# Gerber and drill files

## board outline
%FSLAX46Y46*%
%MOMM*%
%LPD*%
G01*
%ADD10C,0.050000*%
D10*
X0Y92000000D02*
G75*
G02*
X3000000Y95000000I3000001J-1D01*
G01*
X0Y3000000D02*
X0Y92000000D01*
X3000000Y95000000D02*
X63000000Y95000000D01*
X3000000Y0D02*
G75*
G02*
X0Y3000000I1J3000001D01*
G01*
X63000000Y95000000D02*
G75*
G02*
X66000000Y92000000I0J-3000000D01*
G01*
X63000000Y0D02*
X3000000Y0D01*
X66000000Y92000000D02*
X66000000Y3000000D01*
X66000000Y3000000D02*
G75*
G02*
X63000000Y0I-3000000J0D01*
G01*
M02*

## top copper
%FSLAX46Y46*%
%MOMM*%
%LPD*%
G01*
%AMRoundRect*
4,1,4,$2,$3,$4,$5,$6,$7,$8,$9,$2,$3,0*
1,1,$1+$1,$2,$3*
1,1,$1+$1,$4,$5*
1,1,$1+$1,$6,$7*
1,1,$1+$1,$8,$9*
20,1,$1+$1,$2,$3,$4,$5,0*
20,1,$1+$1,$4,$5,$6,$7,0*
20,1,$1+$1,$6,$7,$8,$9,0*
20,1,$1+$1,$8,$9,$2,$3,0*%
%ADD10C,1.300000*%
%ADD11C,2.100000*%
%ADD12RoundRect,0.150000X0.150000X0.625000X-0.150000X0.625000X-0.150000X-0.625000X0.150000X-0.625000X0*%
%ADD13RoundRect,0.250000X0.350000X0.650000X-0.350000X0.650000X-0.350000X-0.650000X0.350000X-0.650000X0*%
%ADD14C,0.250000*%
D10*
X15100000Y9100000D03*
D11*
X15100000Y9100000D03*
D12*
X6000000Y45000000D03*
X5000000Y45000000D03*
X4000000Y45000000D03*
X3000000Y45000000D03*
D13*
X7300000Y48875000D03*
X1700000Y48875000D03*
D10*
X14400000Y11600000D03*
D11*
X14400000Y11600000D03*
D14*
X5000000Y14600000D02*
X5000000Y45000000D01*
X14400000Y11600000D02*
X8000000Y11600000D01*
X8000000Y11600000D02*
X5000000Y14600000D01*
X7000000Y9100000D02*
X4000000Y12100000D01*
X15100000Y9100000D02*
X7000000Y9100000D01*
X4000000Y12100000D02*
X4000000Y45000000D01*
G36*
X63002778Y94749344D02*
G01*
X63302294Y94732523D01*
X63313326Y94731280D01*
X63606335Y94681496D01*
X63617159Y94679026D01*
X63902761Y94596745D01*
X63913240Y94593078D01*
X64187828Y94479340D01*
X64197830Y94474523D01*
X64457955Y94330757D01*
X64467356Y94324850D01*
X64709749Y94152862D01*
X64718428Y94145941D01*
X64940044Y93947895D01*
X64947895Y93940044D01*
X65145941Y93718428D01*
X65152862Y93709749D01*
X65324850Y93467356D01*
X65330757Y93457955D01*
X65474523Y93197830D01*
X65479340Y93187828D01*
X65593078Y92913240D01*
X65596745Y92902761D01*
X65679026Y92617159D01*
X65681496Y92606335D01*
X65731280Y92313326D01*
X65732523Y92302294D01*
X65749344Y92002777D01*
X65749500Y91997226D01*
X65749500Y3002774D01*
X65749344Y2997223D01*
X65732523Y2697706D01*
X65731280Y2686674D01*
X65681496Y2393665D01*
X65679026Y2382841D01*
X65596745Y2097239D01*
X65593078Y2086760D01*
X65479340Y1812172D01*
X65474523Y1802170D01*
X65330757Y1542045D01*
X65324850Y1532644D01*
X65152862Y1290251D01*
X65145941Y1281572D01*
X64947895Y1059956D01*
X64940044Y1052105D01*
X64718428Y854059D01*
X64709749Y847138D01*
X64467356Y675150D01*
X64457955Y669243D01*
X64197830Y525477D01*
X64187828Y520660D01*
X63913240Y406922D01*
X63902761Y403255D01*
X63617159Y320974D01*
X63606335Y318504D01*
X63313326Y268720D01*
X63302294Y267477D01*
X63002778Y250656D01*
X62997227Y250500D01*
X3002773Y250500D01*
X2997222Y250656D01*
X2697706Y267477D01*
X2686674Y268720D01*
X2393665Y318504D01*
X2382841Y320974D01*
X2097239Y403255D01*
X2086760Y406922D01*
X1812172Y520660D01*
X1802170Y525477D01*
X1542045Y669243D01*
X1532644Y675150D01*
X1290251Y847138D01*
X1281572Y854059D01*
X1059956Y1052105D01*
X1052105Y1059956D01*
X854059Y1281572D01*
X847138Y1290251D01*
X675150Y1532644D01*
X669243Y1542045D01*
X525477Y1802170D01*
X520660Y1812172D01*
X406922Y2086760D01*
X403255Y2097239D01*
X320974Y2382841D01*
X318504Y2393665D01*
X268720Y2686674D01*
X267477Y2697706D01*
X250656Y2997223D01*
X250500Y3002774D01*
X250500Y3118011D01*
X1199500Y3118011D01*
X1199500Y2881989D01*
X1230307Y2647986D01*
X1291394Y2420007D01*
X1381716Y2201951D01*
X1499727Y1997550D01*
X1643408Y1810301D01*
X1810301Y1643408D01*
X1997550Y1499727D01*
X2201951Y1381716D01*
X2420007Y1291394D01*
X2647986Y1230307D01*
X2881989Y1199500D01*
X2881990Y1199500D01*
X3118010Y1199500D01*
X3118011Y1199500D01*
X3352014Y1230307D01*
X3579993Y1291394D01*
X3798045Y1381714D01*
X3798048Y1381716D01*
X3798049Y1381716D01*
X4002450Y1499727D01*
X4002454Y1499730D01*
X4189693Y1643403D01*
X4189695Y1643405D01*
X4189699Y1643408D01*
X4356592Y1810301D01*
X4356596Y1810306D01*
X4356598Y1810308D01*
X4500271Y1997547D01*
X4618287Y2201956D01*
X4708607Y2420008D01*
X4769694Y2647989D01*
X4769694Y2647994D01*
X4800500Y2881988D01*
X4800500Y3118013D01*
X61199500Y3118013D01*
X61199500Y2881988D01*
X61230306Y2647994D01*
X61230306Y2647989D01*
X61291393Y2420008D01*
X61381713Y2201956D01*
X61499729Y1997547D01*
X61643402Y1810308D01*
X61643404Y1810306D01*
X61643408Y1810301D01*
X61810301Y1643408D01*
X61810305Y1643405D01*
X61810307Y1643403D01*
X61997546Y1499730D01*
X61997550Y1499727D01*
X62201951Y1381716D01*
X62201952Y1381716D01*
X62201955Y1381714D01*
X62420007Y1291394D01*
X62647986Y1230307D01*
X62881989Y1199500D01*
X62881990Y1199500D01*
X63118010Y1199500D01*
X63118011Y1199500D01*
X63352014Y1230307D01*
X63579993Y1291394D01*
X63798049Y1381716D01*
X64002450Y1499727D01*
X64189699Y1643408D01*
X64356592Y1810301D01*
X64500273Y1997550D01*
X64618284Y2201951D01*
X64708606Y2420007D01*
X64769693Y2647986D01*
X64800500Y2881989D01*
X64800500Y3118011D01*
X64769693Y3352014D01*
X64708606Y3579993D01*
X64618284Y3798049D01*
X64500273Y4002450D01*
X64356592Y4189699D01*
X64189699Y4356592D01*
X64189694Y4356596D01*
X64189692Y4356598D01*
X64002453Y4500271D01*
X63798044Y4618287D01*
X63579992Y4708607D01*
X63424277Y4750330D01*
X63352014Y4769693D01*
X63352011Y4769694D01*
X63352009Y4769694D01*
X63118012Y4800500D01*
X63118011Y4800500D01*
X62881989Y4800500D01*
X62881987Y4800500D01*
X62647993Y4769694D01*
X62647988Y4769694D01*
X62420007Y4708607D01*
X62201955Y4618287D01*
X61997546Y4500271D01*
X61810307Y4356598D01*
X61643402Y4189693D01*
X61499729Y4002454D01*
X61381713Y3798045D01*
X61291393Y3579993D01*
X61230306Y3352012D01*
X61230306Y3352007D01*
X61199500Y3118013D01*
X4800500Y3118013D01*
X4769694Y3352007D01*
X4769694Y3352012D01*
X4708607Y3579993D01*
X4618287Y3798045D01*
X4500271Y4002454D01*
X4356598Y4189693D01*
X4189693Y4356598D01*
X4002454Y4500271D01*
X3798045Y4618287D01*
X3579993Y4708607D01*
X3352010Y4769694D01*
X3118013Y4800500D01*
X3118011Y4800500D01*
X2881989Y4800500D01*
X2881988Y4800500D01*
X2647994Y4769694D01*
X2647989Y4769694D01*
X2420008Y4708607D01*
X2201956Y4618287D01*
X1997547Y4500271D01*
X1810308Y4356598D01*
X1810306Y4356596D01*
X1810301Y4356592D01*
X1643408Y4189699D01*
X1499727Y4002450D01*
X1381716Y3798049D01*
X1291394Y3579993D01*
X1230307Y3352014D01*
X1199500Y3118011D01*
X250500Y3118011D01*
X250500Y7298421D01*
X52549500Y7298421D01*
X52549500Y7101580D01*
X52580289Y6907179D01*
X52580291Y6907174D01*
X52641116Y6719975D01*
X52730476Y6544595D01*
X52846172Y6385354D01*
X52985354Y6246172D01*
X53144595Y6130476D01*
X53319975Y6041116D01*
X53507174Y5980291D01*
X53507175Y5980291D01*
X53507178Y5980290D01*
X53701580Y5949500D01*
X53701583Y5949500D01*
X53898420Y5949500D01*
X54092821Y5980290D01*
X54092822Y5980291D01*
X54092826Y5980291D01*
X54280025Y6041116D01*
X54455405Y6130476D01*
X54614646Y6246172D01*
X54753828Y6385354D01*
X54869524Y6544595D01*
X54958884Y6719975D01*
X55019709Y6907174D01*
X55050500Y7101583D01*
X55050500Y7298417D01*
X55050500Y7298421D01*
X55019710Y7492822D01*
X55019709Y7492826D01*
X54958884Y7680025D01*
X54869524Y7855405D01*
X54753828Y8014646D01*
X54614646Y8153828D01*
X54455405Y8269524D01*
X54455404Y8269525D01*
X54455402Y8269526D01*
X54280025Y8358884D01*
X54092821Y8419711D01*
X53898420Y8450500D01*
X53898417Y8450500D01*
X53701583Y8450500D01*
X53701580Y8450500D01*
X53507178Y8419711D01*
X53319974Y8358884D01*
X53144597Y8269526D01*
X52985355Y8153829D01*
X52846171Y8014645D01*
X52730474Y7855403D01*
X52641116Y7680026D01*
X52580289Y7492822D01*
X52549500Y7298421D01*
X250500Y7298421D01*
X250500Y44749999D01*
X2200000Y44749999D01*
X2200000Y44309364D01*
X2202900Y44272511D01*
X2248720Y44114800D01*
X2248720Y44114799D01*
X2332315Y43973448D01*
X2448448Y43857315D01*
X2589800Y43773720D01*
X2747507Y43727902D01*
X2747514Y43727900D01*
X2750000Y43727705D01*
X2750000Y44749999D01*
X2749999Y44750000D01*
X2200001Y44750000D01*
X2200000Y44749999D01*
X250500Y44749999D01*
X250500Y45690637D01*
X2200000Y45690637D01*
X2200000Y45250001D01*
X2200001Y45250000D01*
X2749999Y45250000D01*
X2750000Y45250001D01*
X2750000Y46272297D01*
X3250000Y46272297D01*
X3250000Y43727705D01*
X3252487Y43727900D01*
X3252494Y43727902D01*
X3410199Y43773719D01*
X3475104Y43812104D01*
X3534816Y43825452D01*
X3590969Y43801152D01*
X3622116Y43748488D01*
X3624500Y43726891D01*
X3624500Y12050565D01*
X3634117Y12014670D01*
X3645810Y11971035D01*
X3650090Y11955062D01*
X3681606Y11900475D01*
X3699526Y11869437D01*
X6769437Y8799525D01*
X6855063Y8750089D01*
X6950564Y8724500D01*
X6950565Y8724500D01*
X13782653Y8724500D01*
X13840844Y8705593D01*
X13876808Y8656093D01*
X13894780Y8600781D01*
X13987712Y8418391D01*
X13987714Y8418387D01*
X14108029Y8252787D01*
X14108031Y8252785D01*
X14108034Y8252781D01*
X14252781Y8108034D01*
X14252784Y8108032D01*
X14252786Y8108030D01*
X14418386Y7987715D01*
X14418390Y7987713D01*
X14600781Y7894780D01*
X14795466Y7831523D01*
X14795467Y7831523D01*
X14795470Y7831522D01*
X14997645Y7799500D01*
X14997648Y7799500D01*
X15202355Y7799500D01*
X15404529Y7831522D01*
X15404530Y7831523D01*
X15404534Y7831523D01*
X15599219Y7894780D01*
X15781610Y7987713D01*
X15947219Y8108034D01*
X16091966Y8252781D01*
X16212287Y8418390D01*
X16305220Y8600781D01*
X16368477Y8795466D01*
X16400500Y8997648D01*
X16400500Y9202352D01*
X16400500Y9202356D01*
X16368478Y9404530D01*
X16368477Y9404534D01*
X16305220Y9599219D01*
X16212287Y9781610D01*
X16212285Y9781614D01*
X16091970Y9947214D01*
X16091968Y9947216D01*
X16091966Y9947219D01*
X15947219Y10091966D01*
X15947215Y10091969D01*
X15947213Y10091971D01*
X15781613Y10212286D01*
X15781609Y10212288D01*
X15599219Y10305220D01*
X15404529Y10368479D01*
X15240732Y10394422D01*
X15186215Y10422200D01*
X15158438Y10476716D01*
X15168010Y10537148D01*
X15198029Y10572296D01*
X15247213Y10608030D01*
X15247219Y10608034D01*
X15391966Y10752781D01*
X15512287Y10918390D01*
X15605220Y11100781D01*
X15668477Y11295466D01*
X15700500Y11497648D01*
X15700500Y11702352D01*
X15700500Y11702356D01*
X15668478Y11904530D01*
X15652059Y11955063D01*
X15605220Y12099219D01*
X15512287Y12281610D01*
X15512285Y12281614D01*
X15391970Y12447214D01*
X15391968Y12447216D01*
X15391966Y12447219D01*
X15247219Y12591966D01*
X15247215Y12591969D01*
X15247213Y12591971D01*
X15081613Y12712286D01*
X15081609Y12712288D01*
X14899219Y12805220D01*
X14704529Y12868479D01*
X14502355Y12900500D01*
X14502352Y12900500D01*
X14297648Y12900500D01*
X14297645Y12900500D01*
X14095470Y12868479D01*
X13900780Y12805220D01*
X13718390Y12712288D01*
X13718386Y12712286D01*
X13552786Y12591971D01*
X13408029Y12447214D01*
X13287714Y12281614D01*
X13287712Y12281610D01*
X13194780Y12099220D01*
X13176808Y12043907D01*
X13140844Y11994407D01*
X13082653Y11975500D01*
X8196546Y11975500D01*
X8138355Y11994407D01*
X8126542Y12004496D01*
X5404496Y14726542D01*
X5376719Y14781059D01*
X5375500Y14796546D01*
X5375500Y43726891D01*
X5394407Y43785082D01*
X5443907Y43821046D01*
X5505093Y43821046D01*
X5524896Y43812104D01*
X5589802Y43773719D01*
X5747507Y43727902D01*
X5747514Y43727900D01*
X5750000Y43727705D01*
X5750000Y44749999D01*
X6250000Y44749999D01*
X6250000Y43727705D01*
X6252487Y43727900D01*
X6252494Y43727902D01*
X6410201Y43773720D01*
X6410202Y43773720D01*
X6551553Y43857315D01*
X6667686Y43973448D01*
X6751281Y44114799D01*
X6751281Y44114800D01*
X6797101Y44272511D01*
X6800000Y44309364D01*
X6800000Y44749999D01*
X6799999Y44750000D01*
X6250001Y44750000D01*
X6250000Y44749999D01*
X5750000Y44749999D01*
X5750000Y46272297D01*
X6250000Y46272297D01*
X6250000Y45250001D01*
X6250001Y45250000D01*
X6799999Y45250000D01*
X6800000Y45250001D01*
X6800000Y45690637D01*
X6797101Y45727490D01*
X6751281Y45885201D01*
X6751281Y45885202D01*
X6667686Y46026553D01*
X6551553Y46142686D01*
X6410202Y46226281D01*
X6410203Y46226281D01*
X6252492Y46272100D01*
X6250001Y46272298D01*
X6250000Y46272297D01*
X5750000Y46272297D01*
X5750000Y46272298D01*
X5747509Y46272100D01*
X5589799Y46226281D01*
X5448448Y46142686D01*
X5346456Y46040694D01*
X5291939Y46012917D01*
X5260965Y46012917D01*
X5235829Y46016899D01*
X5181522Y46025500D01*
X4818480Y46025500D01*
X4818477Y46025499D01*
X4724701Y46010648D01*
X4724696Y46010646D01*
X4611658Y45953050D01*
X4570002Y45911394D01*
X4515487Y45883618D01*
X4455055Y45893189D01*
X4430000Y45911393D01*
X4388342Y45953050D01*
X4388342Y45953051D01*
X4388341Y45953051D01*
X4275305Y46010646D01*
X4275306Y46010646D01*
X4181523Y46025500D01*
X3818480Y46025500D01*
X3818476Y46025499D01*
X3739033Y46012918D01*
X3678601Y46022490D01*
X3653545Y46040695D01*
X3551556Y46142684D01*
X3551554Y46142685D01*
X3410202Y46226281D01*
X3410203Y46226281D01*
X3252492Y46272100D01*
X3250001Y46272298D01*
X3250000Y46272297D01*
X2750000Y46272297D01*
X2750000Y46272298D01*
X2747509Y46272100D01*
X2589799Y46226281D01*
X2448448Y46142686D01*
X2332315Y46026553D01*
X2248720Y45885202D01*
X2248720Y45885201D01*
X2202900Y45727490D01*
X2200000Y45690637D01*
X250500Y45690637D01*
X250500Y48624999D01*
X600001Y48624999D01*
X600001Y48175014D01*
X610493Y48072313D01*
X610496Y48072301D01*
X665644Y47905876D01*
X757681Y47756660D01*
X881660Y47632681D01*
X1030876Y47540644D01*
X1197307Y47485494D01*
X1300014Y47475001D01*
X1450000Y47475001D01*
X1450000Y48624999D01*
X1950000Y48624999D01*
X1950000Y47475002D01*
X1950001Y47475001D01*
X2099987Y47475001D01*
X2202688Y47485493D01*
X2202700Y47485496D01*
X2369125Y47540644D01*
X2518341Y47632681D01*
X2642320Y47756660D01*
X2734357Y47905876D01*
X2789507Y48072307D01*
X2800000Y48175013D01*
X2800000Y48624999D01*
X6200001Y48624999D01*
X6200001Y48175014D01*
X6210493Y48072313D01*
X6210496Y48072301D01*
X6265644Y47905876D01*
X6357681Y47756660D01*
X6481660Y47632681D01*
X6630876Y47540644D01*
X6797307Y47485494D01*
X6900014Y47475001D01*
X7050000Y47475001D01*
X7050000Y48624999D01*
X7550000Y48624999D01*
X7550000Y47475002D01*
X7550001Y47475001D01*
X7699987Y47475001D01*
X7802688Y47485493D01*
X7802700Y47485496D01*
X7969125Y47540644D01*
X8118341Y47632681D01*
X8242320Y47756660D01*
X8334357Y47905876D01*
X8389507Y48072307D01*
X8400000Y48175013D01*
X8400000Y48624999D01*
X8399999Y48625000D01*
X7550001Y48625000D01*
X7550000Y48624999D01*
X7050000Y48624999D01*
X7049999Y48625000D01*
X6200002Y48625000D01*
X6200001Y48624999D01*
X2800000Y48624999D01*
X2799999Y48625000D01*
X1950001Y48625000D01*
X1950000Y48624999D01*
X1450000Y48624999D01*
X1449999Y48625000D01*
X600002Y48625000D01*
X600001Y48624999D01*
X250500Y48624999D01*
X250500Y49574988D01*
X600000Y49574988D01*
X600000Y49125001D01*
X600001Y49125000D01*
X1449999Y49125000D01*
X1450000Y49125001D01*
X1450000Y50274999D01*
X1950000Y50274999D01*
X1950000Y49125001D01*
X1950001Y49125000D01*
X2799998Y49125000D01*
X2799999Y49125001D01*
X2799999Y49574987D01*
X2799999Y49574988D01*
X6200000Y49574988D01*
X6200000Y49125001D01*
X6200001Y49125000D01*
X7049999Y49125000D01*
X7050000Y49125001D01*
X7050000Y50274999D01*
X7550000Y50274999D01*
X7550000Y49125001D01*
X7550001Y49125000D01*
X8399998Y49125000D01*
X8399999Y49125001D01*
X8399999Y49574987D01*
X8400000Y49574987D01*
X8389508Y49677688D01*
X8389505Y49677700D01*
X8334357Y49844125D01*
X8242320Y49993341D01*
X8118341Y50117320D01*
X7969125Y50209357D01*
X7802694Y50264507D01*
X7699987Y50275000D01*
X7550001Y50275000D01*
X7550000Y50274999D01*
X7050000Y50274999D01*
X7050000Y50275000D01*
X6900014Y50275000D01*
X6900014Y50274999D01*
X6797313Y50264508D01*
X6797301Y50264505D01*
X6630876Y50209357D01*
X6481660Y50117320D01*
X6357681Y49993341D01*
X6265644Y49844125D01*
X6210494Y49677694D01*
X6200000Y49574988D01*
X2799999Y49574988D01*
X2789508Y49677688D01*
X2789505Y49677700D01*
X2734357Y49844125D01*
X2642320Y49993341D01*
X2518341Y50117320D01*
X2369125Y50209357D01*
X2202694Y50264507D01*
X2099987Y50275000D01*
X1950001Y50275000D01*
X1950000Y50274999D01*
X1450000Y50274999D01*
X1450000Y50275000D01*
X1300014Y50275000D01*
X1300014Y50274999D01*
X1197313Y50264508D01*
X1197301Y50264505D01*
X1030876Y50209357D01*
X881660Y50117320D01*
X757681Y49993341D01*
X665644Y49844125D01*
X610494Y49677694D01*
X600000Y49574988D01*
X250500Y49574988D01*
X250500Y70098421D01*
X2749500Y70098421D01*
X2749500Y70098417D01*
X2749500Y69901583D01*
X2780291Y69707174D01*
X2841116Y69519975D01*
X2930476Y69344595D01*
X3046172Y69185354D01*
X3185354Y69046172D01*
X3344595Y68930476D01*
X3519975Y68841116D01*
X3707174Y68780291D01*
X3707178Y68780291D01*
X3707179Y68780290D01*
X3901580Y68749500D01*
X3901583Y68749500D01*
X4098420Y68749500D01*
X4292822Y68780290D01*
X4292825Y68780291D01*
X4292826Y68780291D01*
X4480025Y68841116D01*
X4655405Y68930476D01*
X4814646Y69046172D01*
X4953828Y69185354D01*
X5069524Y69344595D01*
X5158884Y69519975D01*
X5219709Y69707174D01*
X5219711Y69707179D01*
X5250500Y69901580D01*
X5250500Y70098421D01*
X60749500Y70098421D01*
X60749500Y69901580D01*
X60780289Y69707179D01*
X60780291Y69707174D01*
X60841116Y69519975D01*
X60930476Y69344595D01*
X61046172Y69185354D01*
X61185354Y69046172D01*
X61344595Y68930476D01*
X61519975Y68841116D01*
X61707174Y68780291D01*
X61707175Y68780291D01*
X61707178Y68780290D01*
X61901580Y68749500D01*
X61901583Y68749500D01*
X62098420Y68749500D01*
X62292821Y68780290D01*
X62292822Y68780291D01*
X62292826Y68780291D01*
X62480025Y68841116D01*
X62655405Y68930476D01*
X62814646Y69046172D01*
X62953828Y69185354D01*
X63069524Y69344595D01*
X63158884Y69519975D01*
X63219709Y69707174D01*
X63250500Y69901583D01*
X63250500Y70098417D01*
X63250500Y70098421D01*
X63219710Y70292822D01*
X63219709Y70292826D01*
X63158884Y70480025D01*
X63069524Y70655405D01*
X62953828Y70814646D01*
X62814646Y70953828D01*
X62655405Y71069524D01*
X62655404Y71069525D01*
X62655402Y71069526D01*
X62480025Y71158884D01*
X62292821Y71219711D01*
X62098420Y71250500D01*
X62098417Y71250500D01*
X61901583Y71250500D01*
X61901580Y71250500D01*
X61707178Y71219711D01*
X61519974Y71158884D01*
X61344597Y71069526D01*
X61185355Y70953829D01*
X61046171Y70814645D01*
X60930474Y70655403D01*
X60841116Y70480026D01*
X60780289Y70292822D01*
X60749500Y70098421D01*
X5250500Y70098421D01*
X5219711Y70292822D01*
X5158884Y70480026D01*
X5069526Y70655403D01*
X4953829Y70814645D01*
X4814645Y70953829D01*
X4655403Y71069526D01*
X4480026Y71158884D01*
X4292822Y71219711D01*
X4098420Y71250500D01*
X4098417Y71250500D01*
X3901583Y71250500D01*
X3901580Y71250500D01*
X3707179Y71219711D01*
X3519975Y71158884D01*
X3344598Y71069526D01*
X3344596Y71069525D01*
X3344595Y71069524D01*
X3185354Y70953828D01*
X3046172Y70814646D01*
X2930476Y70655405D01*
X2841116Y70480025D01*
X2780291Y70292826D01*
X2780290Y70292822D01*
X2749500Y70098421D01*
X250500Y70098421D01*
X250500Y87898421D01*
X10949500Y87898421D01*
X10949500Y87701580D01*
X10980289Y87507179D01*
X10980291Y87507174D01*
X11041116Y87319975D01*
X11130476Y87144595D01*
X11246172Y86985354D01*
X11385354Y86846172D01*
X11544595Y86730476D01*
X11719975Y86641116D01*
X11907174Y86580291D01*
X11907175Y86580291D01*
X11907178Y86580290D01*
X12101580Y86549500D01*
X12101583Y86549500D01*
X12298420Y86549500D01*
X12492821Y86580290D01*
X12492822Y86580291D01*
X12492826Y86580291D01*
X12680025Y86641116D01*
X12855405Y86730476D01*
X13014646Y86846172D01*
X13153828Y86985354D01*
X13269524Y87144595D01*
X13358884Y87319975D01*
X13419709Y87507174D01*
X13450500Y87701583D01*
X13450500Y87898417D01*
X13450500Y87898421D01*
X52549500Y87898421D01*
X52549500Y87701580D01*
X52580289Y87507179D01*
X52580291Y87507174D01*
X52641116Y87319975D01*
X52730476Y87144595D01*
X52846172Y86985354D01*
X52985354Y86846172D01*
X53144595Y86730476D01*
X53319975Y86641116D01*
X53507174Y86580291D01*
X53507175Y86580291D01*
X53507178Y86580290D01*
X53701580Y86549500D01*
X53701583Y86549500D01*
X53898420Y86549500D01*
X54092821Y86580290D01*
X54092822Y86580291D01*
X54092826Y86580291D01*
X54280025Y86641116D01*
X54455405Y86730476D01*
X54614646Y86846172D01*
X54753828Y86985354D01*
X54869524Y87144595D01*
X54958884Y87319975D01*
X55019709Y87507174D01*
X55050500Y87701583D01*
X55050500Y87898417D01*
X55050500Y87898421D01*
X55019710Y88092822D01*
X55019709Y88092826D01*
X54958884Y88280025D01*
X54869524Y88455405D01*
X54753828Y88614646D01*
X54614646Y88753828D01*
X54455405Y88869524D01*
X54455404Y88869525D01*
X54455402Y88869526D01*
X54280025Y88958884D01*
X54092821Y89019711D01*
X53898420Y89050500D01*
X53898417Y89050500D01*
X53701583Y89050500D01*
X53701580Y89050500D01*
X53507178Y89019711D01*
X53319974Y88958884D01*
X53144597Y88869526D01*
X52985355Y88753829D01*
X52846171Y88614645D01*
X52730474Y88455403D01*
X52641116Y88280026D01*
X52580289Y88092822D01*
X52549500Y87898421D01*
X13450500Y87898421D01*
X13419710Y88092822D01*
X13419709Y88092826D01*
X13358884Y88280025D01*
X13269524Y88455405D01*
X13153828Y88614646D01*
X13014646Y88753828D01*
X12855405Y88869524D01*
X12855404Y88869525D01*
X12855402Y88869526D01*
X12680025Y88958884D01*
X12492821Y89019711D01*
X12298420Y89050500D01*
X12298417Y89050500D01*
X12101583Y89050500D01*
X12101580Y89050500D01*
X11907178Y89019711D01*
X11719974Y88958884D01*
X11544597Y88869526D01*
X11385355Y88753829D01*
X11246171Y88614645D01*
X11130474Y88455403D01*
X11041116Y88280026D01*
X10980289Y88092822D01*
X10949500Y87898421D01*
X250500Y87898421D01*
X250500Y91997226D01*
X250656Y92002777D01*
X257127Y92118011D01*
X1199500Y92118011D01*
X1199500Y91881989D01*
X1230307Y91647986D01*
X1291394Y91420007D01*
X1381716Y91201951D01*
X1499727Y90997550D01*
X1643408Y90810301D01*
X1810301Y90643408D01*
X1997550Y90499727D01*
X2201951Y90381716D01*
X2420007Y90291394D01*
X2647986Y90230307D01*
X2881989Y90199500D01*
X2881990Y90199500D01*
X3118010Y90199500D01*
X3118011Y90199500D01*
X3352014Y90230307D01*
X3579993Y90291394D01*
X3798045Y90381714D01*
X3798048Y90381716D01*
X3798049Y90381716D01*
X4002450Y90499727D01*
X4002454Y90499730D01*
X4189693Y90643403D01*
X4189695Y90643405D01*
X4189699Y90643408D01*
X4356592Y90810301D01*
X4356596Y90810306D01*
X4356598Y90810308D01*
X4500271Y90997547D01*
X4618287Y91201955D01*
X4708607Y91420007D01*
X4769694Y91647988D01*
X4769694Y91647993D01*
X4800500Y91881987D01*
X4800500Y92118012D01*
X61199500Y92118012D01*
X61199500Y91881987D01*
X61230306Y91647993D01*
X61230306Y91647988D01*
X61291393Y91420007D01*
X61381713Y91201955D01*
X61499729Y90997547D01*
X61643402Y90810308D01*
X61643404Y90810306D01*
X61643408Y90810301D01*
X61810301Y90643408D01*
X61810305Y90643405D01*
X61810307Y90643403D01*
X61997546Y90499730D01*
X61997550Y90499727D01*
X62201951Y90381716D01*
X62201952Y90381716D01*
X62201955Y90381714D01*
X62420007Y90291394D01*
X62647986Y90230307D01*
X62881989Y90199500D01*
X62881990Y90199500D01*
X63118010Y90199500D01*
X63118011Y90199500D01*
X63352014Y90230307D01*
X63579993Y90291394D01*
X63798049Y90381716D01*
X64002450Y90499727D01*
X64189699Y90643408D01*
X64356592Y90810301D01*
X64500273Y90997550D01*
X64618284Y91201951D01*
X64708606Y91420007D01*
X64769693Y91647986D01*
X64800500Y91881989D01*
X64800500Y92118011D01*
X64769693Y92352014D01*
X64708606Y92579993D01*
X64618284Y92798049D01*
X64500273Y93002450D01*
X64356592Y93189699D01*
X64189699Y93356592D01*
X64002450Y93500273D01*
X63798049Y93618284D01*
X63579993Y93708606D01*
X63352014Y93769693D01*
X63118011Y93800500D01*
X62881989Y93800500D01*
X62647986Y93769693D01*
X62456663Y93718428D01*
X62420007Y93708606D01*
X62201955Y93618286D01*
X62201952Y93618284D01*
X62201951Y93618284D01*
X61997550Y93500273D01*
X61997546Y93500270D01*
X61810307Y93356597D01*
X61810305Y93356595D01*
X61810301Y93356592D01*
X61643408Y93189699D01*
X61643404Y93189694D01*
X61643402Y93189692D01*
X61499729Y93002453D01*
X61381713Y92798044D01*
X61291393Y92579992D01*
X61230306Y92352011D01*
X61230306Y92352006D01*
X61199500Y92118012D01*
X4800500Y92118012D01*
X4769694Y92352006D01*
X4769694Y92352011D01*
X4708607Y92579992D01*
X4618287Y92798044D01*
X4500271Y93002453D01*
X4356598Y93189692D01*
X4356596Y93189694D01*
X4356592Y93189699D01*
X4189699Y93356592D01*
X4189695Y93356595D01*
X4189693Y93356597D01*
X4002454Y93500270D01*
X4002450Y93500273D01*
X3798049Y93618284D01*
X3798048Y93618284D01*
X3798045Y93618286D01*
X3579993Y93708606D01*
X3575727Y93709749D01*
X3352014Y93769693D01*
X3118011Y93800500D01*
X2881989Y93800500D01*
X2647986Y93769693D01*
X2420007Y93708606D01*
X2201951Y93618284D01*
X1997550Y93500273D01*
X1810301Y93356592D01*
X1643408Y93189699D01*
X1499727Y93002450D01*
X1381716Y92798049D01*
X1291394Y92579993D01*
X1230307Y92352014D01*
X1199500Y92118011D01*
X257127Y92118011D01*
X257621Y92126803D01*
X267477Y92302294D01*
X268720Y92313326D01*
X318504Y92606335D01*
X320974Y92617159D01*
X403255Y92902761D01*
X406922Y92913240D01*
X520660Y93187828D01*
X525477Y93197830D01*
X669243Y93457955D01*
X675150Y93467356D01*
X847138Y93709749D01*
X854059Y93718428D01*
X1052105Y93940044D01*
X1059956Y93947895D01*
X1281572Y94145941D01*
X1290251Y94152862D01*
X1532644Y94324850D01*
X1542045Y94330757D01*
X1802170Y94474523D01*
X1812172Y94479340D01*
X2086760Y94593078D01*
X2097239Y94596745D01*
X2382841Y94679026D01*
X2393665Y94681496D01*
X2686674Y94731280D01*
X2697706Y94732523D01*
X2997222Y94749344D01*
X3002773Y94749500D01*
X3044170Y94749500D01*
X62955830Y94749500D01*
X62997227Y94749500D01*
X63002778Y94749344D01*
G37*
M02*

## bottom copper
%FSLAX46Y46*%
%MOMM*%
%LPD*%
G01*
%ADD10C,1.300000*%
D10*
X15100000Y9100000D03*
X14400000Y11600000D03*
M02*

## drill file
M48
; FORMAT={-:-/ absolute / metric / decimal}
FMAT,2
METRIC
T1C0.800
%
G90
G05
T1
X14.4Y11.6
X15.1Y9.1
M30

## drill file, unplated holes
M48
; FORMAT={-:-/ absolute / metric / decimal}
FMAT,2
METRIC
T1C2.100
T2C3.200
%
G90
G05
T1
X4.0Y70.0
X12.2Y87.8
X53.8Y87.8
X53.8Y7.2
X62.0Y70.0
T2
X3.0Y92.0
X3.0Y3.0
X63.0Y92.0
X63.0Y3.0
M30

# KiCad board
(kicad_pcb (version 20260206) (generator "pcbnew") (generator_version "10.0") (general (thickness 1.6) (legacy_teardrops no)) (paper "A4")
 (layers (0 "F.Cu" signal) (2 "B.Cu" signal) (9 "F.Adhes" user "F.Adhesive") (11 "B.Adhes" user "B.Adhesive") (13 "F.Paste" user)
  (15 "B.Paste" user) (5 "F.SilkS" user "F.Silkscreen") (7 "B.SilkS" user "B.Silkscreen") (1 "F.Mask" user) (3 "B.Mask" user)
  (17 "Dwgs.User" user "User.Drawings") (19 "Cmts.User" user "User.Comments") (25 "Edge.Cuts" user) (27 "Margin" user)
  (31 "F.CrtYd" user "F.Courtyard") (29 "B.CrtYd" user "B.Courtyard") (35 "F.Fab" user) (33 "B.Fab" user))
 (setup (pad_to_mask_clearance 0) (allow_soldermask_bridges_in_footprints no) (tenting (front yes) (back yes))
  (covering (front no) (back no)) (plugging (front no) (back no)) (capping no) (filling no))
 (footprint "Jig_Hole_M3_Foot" (layer "F.Cu") (at 54 88)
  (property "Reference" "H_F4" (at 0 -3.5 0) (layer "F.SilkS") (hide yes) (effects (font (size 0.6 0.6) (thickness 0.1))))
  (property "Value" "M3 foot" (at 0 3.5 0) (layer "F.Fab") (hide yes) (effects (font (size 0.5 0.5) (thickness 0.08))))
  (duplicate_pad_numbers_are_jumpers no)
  (pad "" np_thru_hole circle (at 0 0) (size 3.2 3.2) (drill 3.2) (layers "*.Cu" "*.Mask")))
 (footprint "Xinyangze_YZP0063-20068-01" (layer "F.Cu") (at 6.1 81.9)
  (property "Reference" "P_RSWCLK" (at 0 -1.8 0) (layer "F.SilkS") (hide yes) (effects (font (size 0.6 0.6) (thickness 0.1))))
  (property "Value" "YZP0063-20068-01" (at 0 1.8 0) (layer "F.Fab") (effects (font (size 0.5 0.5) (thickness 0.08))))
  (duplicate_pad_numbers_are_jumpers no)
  (pad "1" thru_hole circle (at 0 0) (size 1.3 1.3) (drill 0.8) (layers "*.Cu" "*.Mask") (remove_unused_layers no) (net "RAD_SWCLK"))
  (pad "1" smd circle (at 0 0) (size 2.1 2.1) (layers "F.Cu" "F.Mask" "F.Paste") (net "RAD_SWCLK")))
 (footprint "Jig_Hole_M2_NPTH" (layer "F.Cu") (at 44.8 83.8)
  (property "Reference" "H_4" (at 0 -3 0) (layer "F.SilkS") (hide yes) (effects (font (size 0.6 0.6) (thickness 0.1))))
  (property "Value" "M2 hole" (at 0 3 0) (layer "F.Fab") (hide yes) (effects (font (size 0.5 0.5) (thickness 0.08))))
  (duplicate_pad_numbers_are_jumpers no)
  (pad "" np_thru_hole circle (at 0 0) (size 2.1 2.1) (drill 2.1) (layers "*.Cu" "*.Mask")))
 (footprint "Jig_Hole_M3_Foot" (layer "F.Cu") (at -6 -1)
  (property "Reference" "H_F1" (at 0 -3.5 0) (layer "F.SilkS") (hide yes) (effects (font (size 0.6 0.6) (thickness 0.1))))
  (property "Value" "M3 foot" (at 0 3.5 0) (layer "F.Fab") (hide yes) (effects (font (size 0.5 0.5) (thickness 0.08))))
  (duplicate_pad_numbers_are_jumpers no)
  (pad "" np_thru_hole circle (at 0 0) (size 3.2 3.2) (drill 3.2) (layers "*.Cu" "*.Mask")))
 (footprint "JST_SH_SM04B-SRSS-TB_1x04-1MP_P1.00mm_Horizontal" (layer "F.Cu") (at -4.5 44 180)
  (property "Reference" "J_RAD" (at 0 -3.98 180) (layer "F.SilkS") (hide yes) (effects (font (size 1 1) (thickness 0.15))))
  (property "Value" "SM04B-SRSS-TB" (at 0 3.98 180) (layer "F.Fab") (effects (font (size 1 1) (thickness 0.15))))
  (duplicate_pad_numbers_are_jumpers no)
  (pad "1" smd roundrect (at -1.5 -2 180) (size 0.6 1.55) (layers "F.Cu" "F.Mask" "F.Paste") (roundrect_rratio 0.25) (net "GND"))
  (pad "2" smd roundrect (at -0.5 -2 180) (size 0.6 1.55) (layers "F.Cu" "F.Mask" "F.Paste") (roundrect_rratio 0.25) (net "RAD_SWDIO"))
  (pad "3" smd roundrect (at 0.5 -2 180) (size 0.6 1.55) (layers "F.Cu" "F.Mask" "F.Paste") (roundrect_rratio 0.25) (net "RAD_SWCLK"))
  (pad "4" smd roundrect (at 1.5 -2 180) (size 0.6 1.55) (layers "F.Cu" "F.Mask" "F.Paste") (roundrect_rratio 0.25) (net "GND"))
  (pad "MP" smd roundrect (at -2.8 1.875 180) (size 1.2 1.8) (layers "F.Cu" "F.Mask" "F.Paste") (roundrect_rratio 0.208333) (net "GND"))
  (pad "MP" smd roundrect (at 2.8 1.875 180) (size 1.2 1.8) (layers "F.Cu" "F.Mask" "F.Paste") (roundrect_rratio 0.208333) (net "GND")))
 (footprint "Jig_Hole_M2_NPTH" (layer "F.Cu") (at 3.2 3.2)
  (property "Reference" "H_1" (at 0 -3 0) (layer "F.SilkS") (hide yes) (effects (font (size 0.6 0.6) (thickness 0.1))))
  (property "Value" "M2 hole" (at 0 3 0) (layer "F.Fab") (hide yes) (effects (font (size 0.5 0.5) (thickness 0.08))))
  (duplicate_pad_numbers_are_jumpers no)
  (pad "" np_thru_hole circle (at 0 0) (size 2.1 2.1) (drill 2.1) (layers "*.Cu" "*.Mask")))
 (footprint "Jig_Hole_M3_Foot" (layer "F.Cu") (at 54 -1)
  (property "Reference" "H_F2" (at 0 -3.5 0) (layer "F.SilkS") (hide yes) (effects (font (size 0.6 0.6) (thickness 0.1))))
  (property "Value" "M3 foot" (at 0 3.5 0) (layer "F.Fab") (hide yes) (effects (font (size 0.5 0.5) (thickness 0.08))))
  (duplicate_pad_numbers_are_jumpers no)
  (pad "" np_thru_hole circle (at 0 0) (size 3.2 3.2) (drill 3.2) (layers "*.Cu" "*.Mask")))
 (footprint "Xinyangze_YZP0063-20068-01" (layer "F.Cu") (at 5.4 79.4)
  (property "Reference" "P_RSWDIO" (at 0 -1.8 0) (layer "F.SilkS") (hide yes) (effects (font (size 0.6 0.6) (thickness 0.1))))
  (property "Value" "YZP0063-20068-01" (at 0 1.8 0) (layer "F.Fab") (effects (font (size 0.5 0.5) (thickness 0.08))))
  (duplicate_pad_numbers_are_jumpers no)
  (pad "1" thru_hole circle (at 0 0) (size 1.3 1.3) (drill 0.8) (layers "*.Cu" "*.Mask") (remove_unused_layers no) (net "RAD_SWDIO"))
  (pad "1" smd circle (at 0 0) (size 2.1 2.1) (layers "F.Cu" "F.Mask" "F.Paste") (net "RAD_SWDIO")))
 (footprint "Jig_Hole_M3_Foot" (layer "F.Cu") (at -6 88)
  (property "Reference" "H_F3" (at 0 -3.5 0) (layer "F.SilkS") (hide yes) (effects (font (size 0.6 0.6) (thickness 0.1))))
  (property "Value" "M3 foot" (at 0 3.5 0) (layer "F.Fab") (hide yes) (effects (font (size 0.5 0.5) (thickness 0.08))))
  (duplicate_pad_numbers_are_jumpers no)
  (pad "" np_thru_hole circle (at 0 0) (size 3.2 3.2) (drill 3.2) (layers "*.Cu" "*.Mask")))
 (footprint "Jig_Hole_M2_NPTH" (layer "F.Cu") (at 53 21)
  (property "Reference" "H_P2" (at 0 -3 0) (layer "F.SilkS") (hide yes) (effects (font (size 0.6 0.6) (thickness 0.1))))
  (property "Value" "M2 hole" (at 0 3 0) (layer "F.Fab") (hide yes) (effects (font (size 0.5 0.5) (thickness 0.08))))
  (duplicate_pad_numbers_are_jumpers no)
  (pad "" np_thru_hole circle (at 0 0) (size 2.1 2.1) (drill 2.1) (layers "*.Cu" "*.Mask")))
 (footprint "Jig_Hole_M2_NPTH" (layer "F.Cu") (at -5 21)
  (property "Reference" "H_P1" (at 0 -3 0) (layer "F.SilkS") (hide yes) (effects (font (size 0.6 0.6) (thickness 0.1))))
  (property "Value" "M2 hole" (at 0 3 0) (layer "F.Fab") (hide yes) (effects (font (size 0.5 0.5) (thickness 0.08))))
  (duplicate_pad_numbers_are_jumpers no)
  (pad "" np_thru_hole circle (at 0 0) (size 2.1 2.1) (drill 2.1) (layers "*.Cu" "*.Mask")))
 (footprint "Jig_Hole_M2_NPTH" (layer "F.Cu") (at 44.8 3.2)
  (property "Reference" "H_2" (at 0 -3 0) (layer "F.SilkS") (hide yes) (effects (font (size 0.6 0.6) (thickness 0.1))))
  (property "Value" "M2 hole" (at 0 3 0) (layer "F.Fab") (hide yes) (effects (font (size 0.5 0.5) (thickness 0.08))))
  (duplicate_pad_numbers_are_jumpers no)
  (pad "" np_thru_hole circle (at 0 0) (size 2.1 2.1) (drill 2.1) (layers "*.Cu" "*.Mask")))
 (gr_arc (start -9 -1) (mid -8.12132 -3.12132) (end -6 -4) (stroke (width 0.05) (type default)) (layer "Edge.Cuts"))
 (gr_line (start -9 88) (end -9 -1) (stroke (width 0.05) (type default)) (layer "Edge.Cuts"))
 (gr_line (start -6 -4) (end 54 -4) (stroke (width 0.05) (type default)) (layer "Edge.Cuts"))
 (gr_arc (start -6 91) (mid -8.12132 90.12132) (end -9 88) (stroke (width 0.05) (type default)) (layer "Edge.Cuts"))
 (gr_arc (start 54 -4) (mid 56.12132 -3.12132) (end 57 -1) (stroke (width 0.05) (type default)) (layer "Edge.Cuts"))
 (gr_line (start 54 91) (end -6 91) (stroke (width 0.05) (type default)) (layer "Edge.Cuts"))
 (gr_line (start 57 -1) (end 57 88) (stroke (width 0.05) (type default)) (layer "Edge.Cuts"))
 (gr_arc (start 57 88) (mid 56.12132 90.12132) (end 54 91) (stroke (width 0.05) (type default)) (layer "Edge.Cuts"))
 (segment (start -4 76.4) (end -4 46) (width 0.25) (layer "F.Cu") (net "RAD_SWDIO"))
 (segment (start 5.4 79.4) (end -1 79.4) (width 0.25) (layer "F.Cu") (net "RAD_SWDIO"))
 (segment (start -1 79.4) (end -4 76.4) (width 0.25) (layer "F.Cu") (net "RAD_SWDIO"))
 (segment (start -2 81.9) (end -5 78.9) (width 0.25) (layer "F.Cu") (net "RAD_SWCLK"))
 (segment (start 6.1 81.9) (end -2 81.9) (width 0.25) (layer "F.Cu") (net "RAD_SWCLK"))
 (segment (start -5 78.9) (end -5 46) (width 0.25) (layer "F.Cu") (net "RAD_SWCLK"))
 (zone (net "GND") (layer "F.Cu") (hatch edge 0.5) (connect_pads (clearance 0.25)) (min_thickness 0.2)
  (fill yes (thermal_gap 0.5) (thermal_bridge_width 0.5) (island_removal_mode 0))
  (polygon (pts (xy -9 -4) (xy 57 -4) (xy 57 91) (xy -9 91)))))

